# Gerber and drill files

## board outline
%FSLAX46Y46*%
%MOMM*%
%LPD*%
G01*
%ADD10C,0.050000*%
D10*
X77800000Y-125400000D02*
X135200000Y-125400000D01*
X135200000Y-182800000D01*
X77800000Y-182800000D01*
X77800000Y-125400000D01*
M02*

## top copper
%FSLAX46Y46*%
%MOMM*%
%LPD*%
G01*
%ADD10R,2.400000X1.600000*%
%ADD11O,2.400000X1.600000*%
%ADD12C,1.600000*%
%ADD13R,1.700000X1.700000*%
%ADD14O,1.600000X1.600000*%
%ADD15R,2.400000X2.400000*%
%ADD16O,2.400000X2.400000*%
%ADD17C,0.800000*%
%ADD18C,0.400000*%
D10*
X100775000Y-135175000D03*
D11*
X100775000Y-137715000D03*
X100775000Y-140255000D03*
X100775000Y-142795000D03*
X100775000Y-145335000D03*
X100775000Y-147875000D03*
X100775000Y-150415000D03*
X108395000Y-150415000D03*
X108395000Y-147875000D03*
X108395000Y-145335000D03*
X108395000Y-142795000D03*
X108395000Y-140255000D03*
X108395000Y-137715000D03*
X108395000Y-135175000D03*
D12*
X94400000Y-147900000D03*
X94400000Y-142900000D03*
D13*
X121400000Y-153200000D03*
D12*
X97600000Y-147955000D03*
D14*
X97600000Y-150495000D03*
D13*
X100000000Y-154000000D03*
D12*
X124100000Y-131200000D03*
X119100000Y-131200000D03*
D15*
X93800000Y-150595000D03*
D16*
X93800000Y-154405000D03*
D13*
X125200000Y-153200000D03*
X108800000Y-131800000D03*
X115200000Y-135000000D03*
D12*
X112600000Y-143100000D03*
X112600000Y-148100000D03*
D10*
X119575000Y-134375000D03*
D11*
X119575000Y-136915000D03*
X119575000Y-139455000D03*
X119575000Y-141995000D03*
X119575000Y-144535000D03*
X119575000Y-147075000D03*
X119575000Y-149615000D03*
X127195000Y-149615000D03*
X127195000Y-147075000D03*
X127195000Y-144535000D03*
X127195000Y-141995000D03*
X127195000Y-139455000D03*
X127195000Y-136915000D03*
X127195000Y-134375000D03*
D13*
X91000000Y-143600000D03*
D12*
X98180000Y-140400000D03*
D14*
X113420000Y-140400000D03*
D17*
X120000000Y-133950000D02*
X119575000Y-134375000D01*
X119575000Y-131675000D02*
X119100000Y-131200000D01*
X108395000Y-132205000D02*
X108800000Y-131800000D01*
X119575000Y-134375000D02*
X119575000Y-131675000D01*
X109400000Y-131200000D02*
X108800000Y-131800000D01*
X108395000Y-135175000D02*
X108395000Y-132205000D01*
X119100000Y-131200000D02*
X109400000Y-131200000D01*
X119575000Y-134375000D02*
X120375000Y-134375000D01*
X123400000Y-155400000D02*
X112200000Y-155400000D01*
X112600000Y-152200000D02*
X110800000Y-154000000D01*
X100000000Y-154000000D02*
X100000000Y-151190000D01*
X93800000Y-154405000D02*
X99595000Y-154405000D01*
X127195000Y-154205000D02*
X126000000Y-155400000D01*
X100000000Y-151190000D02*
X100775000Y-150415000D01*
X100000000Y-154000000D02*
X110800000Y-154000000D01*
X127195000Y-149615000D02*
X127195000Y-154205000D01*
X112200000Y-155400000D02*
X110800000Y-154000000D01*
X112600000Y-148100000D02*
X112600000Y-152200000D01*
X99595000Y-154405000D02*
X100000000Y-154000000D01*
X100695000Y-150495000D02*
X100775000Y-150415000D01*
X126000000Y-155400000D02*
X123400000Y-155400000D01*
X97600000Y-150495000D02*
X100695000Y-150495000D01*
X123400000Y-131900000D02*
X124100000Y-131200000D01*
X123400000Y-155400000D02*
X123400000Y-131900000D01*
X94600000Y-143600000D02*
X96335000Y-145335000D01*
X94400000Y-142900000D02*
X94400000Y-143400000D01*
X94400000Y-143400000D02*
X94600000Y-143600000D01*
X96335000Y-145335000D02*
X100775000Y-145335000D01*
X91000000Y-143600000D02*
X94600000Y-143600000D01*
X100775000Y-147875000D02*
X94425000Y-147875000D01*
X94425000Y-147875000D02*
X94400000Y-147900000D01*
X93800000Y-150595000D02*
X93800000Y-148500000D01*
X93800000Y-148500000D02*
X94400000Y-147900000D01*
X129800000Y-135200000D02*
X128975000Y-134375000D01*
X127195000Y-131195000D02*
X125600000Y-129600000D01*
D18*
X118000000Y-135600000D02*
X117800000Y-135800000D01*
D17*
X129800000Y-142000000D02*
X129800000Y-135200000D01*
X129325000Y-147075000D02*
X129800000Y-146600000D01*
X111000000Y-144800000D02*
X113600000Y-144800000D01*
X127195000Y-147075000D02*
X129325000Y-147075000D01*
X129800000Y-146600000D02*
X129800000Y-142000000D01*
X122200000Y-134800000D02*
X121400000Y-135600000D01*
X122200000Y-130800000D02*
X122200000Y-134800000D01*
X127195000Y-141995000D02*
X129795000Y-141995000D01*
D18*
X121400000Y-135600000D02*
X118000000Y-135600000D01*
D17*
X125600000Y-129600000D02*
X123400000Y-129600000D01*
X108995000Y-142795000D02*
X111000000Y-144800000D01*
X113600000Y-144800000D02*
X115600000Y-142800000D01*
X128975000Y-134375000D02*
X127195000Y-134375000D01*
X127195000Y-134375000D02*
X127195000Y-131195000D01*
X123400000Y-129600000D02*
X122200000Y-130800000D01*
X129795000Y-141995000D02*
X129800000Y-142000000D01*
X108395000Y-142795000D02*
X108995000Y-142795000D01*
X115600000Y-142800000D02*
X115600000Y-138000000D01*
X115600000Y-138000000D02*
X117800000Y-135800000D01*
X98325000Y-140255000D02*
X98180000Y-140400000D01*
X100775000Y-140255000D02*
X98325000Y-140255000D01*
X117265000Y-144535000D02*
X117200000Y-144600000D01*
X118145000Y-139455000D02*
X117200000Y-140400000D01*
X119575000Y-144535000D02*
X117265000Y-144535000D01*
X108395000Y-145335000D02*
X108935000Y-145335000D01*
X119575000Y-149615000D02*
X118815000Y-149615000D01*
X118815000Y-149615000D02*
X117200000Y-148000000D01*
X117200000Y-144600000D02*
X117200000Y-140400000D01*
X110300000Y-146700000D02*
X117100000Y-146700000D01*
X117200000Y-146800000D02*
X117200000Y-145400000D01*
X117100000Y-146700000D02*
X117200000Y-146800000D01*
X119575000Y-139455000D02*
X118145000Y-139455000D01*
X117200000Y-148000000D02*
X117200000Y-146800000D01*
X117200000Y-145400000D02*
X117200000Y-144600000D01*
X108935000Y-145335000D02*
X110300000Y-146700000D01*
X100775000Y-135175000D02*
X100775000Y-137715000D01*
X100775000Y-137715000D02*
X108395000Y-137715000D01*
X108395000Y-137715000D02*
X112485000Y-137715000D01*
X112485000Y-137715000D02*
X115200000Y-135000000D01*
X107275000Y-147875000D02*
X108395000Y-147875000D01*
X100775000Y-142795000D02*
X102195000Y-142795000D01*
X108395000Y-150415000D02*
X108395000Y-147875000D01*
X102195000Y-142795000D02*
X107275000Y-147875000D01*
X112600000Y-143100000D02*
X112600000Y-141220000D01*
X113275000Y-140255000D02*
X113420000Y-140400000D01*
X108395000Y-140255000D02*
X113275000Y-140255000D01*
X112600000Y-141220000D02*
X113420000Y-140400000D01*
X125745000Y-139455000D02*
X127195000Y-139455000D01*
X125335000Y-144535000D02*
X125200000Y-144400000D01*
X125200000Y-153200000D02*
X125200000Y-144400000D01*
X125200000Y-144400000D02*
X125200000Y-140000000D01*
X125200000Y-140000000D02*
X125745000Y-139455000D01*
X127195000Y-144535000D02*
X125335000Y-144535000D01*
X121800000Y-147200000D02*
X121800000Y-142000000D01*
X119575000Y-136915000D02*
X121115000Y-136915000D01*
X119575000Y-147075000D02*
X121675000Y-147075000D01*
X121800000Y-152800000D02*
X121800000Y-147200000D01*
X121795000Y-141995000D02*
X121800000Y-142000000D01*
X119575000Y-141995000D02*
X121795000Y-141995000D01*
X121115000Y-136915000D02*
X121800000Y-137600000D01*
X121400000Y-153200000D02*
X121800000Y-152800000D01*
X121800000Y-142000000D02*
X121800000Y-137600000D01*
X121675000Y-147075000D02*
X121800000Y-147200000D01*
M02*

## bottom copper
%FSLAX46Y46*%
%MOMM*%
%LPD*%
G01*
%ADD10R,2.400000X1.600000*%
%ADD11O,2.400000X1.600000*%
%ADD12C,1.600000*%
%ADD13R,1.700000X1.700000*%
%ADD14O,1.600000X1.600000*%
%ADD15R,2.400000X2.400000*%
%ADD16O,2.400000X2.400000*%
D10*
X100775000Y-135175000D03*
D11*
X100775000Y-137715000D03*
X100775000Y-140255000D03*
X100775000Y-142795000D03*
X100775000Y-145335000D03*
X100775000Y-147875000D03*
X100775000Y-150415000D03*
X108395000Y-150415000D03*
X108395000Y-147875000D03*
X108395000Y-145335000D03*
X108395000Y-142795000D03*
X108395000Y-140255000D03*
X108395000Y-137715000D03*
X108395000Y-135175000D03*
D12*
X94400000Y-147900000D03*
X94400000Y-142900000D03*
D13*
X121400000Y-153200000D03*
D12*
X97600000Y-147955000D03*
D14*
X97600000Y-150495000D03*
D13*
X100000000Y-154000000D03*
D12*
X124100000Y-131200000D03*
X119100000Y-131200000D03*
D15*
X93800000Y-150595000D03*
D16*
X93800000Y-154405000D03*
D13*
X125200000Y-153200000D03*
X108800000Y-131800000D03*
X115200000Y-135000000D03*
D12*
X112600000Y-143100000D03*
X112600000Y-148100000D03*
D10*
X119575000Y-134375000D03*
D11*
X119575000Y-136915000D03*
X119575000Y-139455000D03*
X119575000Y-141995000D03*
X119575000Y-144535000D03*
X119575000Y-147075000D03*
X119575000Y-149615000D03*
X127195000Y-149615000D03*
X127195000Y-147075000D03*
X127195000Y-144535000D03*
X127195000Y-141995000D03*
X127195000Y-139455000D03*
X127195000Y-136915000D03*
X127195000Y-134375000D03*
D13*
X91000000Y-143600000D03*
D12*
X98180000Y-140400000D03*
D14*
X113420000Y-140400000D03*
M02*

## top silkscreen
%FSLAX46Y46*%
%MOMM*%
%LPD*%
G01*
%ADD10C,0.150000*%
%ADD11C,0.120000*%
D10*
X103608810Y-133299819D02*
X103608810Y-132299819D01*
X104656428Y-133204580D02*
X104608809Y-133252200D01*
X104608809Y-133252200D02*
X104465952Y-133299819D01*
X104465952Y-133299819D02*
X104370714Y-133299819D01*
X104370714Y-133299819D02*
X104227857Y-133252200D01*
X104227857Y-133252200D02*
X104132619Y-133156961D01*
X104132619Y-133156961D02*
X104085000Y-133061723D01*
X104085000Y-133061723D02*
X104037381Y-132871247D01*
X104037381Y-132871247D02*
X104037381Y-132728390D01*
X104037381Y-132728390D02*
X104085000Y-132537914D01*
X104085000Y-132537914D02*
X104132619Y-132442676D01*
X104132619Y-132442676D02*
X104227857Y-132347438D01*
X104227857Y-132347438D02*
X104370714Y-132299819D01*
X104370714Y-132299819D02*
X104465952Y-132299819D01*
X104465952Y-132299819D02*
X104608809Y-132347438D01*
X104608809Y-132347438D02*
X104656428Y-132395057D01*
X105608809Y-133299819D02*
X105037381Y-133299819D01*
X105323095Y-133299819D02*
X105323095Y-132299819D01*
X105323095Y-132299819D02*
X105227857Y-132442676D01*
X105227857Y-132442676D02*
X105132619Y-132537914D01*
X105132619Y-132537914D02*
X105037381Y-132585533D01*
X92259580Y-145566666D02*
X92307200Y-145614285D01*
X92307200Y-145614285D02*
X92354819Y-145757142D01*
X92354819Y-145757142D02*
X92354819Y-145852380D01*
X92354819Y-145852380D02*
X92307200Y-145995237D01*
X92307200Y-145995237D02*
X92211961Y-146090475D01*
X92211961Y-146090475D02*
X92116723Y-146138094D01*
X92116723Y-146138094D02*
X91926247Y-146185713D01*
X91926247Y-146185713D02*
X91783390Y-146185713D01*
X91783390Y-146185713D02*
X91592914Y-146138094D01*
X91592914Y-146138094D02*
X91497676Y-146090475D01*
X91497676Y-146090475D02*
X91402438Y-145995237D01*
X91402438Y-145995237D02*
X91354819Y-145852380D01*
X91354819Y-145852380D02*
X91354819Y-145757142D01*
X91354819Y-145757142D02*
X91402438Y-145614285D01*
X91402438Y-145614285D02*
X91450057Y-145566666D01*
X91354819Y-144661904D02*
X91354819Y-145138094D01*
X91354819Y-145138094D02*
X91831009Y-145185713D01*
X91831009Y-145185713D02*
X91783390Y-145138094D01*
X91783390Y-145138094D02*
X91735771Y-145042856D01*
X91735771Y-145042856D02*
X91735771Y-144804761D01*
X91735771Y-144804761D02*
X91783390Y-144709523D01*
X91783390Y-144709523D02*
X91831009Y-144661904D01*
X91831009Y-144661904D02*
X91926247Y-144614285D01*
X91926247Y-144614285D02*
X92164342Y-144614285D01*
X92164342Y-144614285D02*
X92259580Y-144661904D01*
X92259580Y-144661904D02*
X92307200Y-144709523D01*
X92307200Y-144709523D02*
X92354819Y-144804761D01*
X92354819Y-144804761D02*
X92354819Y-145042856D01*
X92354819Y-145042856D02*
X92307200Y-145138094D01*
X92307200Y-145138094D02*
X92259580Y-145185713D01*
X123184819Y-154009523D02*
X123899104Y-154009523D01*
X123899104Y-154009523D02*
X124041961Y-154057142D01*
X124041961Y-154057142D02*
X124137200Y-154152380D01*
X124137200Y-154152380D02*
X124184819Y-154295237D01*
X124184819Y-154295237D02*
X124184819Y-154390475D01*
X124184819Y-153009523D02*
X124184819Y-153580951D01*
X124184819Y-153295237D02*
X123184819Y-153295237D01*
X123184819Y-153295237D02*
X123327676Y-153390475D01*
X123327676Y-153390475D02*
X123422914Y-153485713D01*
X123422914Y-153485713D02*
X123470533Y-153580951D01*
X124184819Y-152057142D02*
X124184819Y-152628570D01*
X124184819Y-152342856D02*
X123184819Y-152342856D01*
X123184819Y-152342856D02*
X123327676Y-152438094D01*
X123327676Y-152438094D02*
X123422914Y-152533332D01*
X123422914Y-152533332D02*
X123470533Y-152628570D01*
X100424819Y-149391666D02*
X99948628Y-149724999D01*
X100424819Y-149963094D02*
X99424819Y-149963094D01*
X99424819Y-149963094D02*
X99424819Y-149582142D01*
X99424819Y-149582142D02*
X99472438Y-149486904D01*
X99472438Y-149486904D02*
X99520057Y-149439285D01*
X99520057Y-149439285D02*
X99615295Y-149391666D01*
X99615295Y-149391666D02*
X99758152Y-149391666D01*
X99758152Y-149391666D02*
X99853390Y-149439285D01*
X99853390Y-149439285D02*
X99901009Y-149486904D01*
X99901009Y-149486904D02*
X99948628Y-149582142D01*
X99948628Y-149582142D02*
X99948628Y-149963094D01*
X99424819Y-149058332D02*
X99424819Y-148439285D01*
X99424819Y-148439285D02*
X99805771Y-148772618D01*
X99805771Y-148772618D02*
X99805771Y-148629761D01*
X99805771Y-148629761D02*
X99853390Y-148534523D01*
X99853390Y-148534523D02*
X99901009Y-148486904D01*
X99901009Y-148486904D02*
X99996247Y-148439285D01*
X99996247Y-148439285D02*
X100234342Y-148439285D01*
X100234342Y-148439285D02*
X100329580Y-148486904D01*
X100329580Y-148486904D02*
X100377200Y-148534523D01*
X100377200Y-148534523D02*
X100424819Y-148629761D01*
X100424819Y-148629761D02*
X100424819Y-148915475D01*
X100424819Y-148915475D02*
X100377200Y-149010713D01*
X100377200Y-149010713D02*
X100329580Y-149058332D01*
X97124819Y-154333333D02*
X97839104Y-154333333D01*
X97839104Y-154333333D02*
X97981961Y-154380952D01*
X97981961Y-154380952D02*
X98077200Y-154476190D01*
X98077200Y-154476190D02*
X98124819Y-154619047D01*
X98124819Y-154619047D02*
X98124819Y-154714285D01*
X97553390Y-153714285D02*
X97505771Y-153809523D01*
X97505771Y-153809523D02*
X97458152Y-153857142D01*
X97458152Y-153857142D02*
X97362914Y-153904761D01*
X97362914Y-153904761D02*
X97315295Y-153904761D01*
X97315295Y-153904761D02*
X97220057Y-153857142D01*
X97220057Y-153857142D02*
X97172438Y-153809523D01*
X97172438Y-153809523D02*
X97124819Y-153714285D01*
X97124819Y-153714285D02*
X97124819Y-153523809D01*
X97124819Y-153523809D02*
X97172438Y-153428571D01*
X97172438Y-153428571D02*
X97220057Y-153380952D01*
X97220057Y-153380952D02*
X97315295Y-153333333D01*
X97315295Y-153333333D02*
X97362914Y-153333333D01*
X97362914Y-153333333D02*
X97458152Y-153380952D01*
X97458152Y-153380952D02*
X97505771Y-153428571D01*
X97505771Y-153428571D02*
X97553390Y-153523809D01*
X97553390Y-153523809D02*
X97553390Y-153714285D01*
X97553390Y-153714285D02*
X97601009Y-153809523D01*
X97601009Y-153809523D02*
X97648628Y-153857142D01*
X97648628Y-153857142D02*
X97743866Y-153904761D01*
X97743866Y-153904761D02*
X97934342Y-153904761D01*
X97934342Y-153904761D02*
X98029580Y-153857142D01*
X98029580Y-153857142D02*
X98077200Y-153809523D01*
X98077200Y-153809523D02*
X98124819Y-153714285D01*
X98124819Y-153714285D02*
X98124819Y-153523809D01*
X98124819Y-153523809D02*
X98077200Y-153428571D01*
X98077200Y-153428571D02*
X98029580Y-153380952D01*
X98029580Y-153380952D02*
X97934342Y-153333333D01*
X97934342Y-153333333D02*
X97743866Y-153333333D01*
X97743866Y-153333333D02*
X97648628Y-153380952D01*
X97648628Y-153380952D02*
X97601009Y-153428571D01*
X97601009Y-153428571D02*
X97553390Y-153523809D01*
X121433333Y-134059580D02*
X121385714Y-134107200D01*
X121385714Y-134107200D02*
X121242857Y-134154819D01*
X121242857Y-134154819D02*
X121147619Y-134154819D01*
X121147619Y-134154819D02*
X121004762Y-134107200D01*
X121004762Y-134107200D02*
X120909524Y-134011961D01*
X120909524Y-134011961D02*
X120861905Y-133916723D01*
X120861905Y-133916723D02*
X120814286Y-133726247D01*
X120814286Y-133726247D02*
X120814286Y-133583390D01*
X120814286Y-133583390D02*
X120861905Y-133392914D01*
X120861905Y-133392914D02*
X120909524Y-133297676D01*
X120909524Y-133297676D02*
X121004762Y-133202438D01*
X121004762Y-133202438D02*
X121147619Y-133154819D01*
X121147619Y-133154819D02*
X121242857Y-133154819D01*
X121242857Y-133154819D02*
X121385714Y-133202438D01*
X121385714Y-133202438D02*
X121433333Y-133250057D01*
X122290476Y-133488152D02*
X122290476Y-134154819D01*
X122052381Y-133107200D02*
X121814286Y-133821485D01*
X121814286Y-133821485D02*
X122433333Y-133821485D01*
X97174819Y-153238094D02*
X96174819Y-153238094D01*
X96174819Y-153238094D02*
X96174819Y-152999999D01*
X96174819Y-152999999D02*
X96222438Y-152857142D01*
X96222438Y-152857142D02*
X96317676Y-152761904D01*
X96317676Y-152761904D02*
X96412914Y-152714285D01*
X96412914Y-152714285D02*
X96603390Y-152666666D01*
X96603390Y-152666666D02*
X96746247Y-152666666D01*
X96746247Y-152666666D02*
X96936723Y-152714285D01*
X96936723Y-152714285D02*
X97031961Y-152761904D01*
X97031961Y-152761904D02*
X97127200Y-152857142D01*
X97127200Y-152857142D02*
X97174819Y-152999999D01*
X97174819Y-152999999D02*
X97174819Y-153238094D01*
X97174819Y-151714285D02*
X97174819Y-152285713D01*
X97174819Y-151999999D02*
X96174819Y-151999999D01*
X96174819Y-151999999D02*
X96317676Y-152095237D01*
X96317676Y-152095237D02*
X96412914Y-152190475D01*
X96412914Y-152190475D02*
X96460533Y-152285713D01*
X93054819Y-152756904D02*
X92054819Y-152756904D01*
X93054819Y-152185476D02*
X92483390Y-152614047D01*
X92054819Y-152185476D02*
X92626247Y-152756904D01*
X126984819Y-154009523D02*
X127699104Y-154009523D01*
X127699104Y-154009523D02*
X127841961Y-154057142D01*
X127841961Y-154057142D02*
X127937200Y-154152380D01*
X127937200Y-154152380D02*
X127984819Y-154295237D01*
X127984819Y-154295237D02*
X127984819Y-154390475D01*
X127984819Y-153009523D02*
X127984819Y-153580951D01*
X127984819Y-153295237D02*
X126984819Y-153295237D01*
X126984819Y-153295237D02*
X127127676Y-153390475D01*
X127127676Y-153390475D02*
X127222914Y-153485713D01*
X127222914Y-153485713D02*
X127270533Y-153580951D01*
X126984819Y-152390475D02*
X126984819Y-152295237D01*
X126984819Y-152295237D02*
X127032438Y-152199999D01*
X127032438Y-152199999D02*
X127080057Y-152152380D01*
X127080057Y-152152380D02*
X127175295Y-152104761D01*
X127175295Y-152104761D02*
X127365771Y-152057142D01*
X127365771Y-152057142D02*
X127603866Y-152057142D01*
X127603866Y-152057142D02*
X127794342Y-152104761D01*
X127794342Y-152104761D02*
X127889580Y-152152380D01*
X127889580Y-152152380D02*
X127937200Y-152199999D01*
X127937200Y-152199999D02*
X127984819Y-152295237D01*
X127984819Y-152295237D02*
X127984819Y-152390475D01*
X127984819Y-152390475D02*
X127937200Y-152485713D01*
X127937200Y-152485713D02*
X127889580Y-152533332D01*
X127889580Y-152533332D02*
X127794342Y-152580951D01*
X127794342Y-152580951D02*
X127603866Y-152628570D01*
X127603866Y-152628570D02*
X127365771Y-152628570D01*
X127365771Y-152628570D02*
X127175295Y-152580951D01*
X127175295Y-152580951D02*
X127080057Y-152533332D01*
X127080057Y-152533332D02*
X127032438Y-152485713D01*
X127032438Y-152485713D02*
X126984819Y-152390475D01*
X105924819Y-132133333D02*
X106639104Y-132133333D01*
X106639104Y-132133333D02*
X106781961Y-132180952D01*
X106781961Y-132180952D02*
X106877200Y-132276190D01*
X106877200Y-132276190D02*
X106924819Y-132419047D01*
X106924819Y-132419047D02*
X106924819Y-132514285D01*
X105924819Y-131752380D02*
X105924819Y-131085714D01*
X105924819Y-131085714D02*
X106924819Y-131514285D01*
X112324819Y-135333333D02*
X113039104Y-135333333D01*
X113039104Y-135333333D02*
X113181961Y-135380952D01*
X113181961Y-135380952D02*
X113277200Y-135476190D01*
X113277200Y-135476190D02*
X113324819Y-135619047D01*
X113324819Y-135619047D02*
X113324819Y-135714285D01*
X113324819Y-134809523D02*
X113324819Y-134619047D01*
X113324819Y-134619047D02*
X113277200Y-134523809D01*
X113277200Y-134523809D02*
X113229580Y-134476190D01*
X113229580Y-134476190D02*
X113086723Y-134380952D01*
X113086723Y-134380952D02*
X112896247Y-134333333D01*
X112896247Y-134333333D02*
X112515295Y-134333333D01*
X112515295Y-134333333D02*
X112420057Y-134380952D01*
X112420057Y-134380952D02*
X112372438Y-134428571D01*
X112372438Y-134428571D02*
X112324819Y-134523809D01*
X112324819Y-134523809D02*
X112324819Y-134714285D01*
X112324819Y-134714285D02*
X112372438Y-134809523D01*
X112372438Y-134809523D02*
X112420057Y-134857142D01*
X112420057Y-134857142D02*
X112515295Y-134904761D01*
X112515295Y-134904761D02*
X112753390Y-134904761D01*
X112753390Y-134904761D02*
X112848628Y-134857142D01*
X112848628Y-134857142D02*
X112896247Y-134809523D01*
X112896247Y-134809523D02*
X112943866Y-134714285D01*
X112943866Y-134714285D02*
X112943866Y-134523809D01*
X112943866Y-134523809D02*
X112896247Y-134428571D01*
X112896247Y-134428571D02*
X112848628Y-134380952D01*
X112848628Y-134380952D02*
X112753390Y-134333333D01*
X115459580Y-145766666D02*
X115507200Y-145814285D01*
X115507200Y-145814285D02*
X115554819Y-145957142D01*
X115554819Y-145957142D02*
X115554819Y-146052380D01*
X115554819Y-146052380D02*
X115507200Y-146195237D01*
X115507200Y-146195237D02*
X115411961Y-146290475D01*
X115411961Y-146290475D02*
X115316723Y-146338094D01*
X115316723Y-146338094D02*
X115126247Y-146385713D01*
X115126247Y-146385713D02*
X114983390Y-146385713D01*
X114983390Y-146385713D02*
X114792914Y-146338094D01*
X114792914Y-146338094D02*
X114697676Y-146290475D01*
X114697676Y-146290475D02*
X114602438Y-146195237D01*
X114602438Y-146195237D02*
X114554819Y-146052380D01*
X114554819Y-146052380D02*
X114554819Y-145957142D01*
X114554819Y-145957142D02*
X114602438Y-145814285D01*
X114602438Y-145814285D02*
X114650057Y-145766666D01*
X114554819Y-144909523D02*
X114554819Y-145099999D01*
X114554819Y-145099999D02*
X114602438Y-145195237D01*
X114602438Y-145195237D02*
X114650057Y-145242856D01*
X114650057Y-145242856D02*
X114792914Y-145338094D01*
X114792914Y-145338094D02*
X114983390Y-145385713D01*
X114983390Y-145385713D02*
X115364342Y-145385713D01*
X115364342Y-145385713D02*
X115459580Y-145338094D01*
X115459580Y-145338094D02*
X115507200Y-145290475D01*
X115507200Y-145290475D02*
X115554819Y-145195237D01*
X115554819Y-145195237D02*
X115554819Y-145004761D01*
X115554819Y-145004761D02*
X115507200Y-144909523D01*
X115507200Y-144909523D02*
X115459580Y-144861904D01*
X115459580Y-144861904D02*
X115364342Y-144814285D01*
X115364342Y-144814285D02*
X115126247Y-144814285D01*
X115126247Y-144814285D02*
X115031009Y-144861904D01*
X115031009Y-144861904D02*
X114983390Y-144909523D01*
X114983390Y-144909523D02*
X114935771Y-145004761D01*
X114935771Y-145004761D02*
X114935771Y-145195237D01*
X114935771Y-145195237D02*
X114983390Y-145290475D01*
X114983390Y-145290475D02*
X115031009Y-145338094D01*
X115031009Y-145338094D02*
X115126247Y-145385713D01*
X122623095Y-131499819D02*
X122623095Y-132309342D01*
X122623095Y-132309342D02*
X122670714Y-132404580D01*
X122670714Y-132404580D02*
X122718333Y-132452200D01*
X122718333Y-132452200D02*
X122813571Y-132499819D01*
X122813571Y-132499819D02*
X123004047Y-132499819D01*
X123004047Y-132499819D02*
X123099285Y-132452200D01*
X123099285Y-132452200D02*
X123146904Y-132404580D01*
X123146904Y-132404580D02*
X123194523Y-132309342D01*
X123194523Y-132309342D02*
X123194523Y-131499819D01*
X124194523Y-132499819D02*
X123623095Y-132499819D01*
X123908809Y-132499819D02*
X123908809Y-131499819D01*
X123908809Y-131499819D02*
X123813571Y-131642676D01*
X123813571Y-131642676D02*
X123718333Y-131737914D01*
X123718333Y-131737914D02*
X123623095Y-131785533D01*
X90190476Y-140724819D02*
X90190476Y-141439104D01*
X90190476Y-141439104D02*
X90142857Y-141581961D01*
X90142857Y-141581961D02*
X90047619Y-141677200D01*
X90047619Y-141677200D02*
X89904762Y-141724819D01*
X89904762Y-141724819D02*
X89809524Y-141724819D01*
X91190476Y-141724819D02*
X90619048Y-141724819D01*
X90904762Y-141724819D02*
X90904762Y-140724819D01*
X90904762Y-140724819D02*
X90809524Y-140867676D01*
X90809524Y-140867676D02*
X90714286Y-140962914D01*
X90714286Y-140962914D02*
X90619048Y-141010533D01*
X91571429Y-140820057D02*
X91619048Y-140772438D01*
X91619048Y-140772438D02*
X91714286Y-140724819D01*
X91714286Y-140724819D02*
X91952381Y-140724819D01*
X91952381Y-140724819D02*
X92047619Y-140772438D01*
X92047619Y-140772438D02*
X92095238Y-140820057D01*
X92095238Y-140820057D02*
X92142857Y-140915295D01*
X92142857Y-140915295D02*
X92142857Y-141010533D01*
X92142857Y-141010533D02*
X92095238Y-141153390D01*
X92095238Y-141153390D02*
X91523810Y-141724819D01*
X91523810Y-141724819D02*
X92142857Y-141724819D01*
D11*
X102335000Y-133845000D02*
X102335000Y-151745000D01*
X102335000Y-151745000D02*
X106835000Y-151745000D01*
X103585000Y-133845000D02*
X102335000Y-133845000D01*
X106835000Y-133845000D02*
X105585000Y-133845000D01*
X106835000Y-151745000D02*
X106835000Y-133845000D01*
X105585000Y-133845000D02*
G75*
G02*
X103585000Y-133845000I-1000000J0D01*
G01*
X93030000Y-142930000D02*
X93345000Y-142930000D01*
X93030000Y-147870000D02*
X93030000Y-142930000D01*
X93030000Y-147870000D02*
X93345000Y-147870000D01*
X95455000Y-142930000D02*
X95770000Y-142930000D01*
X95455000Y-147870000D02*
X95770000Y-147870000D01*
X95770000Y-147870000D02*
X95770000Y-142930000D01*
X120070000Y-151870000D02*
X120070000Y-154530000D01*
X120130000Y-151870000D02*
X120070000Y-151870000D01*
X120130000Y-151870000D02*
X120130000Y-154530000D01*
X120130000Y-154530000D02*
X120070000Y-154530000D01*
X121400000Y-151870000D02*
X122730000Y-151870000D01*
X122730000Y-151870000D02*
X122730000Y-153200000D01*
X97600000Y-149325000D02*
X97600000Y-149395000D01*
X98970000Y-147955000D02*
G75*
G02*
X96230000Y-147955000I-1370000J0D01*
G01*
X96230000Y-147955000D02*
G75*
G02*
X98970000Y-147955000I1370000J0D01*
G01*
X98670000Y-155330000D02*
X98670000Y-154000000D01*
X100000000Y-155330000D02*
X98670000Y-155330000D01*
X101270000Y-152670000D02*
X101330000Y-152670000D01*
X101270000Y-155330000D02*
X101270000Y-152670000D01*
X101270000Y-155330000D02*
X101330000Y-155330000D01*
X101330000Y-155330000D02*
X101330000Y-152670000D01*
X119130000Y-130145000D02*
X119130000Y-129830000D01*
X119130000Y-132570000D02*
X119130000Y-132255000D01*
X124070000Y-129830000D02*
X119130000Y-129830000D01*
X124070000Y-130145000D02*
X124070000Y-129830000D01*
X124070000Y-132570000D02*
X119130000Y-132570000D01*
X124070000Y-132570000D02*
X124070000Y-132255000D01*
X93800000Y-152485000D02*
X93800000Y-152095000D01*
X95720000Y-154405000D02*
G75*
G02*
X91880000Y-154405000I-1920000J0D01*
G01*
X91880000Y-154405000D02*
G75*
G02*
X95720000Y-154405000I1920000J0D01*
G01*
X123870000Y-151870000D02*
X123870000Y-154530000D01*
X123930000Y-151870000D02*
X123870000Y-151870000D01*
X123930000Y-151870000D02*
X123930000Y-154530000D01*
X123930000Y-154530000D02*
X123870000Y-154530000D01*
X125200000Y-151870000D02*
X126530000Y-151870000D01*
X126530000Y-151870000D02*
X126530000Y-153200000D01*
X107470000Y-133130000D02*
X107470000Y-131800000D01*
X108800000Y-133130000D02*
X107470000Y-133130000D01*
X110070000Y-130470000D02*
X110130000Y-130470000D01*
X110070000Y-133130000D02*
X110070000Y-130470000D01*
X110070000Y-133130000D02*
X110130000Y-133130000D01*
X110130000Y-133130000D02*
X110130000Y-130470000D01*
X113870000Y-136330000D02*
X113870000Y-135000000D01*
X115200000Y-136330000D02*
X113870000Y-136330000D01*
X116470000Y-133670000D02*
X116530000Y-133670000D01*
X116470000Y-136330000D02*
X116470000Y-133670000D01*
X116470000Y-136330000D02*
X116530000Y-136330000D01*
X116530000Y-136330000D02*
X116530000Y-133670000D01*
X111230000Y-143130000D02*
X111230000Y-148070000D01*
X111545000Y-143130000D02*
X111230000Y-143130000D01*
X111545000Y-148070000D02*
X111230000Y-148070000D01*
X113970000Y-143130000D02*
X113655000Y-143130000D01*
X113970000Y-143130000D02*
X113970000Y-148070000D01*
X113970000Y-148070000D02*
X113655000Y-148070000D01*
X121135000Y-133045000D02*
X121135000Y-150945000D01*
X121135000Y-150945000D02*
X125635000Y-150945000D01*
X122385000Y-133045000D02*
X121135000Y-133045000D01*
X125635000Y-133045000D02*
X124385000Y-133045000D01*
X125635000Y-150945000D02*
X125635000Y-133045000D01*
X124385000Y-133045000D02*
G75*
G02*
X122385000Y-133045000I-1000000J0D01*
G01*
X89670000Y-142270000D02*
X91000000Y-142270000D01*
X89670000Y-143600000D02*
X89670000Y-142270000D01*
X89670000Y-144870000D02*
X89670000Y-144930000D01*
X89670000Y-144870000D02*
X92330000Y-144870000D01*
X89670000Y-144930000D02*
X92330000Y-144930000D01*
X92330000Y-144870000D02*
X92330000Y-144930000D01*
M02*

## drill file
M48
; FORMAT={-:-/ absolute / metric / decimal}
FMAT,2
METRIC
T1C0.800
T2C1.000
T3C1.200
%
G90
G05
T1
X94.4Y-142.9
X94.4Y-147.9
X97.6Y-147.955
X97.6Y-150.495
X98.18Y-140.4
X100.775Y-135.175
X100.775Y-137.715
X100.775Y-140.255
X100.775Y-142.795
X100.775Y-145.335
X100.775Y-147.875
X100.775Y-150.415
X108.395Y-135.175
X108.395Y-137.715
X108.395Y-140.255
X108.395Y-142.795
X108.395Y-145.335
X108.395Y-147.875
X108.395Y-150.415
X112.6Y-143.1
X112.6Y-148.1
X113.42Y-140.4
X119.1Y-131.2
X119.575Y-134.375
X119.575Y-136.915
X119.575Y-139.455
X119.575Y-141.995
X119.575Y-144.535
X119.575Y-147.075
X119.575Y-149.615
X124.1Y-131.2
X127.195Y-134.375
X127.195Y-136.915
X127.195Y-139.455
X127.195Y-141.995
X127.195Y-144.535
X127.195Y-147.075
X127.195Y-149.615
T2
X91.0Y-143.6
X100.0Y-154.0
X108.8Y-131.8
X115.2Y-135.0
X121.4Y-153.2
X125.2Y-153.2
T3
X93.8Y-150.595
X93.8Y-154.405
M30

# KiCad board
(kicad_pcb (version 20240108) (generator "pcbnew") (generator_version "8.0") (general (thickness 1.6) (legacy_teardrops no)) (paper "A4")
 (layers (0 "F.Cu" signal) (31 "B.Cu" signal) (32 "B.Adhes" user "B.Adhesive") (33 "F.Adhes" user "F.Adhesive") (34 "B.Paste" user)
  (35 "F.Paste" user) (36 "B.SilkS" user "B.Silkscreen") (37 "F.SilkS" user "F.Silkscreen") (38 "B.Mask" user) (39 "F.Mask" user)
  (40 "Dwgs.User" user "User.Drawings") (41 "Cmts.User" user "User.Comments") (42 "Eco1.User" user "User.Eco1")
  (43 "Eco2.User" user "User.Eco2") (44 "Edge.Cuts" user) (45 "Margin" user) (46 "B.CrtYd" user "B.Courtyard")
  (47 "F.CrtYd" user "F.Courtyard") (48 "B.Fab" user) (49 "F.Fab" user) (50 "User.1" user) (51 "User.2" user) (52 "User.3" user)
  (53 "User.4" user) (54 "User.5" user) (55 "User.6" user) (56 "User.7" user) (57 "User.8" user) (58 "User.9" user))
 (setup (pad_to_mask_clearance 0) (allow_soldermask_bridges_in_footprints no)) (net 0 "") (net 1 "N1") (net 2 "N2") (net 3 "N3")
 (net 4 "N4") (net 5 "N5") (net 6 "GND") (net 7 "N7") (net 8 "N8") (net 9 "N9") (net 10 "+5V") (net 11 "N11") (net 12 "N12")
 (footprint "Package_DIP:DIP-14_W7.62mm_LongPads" (layer "F.Cu") (at 100.775 135.175)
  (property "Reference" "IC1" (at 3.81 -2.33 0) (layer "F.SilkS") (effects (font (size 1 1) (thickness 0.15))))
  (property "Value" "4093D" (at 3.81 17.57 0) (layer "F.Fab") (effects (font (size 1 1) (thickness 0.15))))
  (fp_line (start 1.56 -1.33) (end 1.56 16.57) (stroke (width 0.12) (type solid)) (layer "F.SilkS"))
  (fp_line (start 1.56 16.57) (end 6.06 16.57) (stroke (width 0.12) (type solid)) (layer "F.SilkS"))
  (fp_line (start 2.81 -1.33) (end 1.56 -1.33) (stroke (width 0.12) (type solid)) (layer "F.SilkS"))
  (fp_line (start 6.06 -1.33) (end 4.81 -1.33) (stroke (width 0.12) (type solid)) (layer "F.SilkS"))
  (fp_line (start 6.06 16.57) (end 6.06 -1.33) (stroke (width 0.12) (type solid)) (layer "F.SilkS"))
  (fp_arc (start 4.81 -1.33) (mid 3.81 -0.33) (end 2.81 -1.33) (stroke (width 0.12) (type solid)) (layer "F.SilkS"))
  (pad "1" thru_hole rect (at 0 0) (size 2.4 1.6) (drill 0.8) (layers "*.Cu" "*.Mask") (remove_unused_layers no) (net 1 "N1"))
  (pad "2" thru_hole oval (at 0 2.54) (size 2.4 1.6) (drill 0.8) (layers "*.Cu" "*.Mask") (remove_unused_layers no) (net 1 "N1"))
  (pad "3" thru_hole oval (at 0 5.08) (size 2.4 1.6) (drill 0.8) (layers "*.Cu" "*.Mask") (remove_unused_layers no) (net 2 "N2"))
  (pad "4" thru_hole oval (at 0 7.62) (size 2.4 1.6) (drill 0.8) (layers "*.Cu" "*.Mask") (remove_unused_layers no) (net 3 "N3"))
  (pad "5" thru_hole oval (at 0 10.16) (size 2.4 1.6) (drill 0.8) (layers "*.Cu" "*.Mask") (remove_unused_layers no) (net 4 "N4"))
  (pad "6" thru_hole oval (at 0 12.7) (size 2.4 1.6) (drill 0.8) (layers "*.Cu" "*.Mask") (remove_unused_layers no) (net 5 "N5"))
  (pad "7" thru_hole oval (at 0 15.24) (size 2.4 1.6) (drill 0.8) (layers "*.Cu" "*.Mask") (remove_unused_layers no) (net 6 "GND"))
  (pad "8" thru_hole oval (at 7.62 15.24) (size 2.4 1.6) (drill 0.8) (layers "*.Cu" "*.Mask") (remove_unused_layers no) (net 3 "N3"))
  (pad "9" thru_hole oval (at 7.62 12.7) (size 2.4 1.6) (drill 0.8) (layers "*.Cu" "*.Mask") (remove_unused_layers no) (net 3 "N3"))
  (pad "10" thru_hole oval (at 7.62 10.16) (size 2.4 1.6) (drill 0.8) (layers "*.Cu" "*.Mask") (remove_unused_layers no) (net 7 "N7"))
  (pad "11" thru_hole oval (at 7.62 7.62) (size 2.4 1.6) (drill 0.8) (layers "*.Cu" "*.Mask") (remove_unused_layers no) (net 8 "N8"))
  (pad "12" thru_hole oval (at 7.62 5.08) (size 2.4 1.6) (drill 0.8) (layers "*.Cu" "*.Mask") (remove_unused_layers no) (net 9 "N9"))
  (pad "13" thru_hole oval (at 7.62 2.54) (size 2.4 1.6) (drill 0.8) (layers "*.Cu" "*.Mask") (remove_unused_layers no) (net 1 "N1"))
  (pad "14" thru_hole oval (at 7.62 0) (size 2.4 1.6) (drill 0.8) (layers "*.Cu" "*.Mask") (remove_unused_layers no) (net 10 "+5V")))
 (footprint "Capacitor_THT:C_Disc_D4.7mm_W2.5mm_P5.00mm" (layer "F.Cu") (at 94.4 147.9 90)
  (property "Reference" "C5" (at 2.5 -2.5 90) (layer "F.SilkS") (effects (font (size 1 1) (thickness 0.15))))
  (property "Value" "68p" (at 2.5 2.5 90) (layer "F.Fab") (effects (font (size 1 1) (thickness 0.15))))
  (fp_line (start 4.97 -1.37) (end 4.97 -1.055) (stroke (width 0.12) (type solid)) (layer "F.SilkS"))
  (fp_line (start 0.03 -1.37) (end 4.97 -1.37) (stroke (width 0.12) (type solid)) (layer "F.SilkS"))
  (fp_line (start 0.03 -1.37) (end 0.03 -1.055) (stroke (width 0.12) (type solid)) (layer "F.SilkS"))
  (fp_line (start 4.97 1.055) (end 4.97 1.37) (stroke (width 0.12) (type solid)) (layer "F.SilkS"))
  (fp_line (start 0.03 1.055) (end 0.03 1.37) (stroke (width 0.12) (type solid)) (layer "F.SilkS"))
  (fp_line (start 0.03 1.37) (end 4.97 1.37) (stroke (width 0.12) (type solid)) (layer "F.SilkS"))
  (pad "1" thru_hole circle (at 0 0 90) (size 1.6 1.6) (drill 0.8) (layers "*.Cu" "*.Mask") (remove_unused_layers no) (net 5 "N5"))
  (pad "2" thru_hole circle (at 5 0 90) (size 1.6 1.6) (drill 0.8) (layers "*.Cu" "*.Mask") (remove_unused_layers no) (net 4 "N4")))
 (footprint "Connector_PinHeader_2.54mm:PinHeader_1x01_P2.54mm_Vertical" (layer "F.Cu") (at 121.4 153.2 -90)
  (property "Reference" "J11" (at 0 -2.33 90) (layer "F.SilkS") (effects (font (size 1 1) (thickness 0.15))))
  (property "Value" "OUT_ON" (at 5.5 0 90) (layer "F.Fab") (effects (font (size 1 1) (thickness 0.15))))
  (fp_line (start -1.33 1.33) (end 1.33 1.33) (stroke (width 0.12) (type solid)) (layer "F.SilkS"))
  (fp_line (start -1.33 1.27) (end -1.33 1.33) (stroke (width 0.12) (type solid)) (layer "F.SilkS"))
  (fp_line (start -1.33 1.27) (end 1.33 1.27) (stroke (width 0.12) (type solid)) (layer "F.SilkS"))
  (fp_line (start 1.33 1.27) (end 1.33 1.33) (stroke (width 0.12) (type solid)) (layer "F.SilkS"))
  (fp_line (start -1.33 0) (end -1.33 -1.33) (stroke (width 0.12) (type solid)) (layer "F.SilkS"))
  (fp_line (start -1.33 -1.33) (end 0 -1.33) (stroke (width 0.12) (type solid)) (layer "F.SilkS"))
  (pad "1" thru_hole rect (at 0 0 270) (size 1.7 1.7) (drill 1) (layers "*.Cu" "*.Mask") (remove_unused_layers no) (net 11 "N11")))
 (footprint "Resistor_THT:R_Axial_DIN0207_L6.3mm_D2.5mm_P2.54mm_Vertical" (layer "F.Cu") (at 97.6 147.955 -90)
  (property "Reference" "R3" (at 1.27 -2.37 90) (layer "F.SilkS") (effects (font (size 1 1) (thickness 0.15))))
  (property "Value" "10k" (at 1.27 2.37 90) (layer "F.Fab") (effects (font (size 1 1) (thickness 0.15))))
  (fp_line (start 1.37 0) (end 1.44 0) (stroke (width 0.12) (type solid)) (layer "F.SilkS"))
  (fp_circle (center 0 0) (end 1.37 0) (stroke (width 0.12) (type solid)) (fill none) (layer "F.SilkS"))
  (pad "1" thru_hole circle (at 0 0 270) (size 1.6 1.6) (drill 0.8) (layers "*.Cu" "*.Mask") (remove_unused_layers no) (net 5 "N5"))
  (pad "2" thru_hole oval (at 2.54 0 270) (size 1.6 1.6) (drill 0.8) (layers "*.Cu" "*.Mask") (remove_unused_layers no) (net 6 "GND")))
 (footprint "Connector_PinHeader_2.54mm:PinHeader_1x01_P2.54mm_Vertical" (layer "F.Cu") (at 100 154 90)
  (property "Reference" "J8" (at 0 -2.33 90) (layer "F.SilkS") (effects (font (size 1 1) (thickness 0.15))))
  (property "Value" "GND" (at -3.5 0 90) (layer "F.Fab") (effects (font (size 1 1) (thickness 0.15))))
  (fp_line (start -1.33 -1.33) (end 0 -1.33) (stroke (width 0.12) (type solid)) (layer "F.SilkS"))
  (fp_line (start -1.33 0) (end -1.33 -1.33) (stroke (width 0.12) (type solid)) (layer "F.SilkS"))
  (fp_line (start 1.33 1.27) (end 1.33 1.33) (stroke (width 0.12) (type solid)) (layer "F.SilkS"))
  (fp_line (start -1.33 1.27) (end 1.33 1.27) (stroke (width 0.12) (type solid)) (layer "F.SilkS"))
  (fp_line (start -1.33 1.27) (end -1.33 1.33) (stroke (width 0.12) (type solid)) (layer "F.SilkS"))
  (fp_line (start -1.33 1.33) (end 1.33 1.33) (stroke (width 0.12) (type solid)) (layer "F.SilkS"))
  (pad "1" thru_hole rect (at 0 0 90) (size 1.7 1.7) (drill 1) (layers "*.Cu" "*.Mask") (remove_unused_layers no) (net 6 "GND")))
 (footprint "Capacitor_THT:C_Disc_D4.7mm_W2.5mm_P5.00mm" (layer "F.Cu") (at 124.1 131.2 180)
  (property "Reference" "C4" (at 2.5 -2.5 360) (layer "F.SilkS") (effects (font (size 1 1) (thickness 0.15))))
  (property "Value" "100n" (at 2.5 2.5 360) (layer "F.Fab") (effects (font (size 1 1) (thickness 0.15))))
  (fp_line (start 4.97 1.055) (end 4.97 1.37) (stroke (width 0.12) (type solid)) (layer "F.SilkS"))
  (fp_line (start 4.97 -1.37) (end 4.97 -1.055) (stroke (width 0.12) (type solid)) (layer "F.SilkS"))
  (fp_line (start 0.03 1.37) (end 4.97 1.37) (stroke (width 0.12) (type solid)) (layer "F.SilkS"))
  (fp_line (start 0.03 1.055) (end 0.03 1.37) (stroke (width 0.12) (type solid)) (layer "F.SilkS"))
  (fp_line (start 0.03 -1.37) (end 4.97 -1.37) (stroke (width 0.12) (type solid)) (layer "F.SilkS"))
  (fp_line (start 0.03 -1.37) (end 0.03 -1.055) (stroke (width 0.12) (type solid)) (layer "F.SilkS"))
  (pad "1" thru_hole circle (at 0 0 180) (size 1.6 1.6) (drill 0.8) (layers "*.Cu" "*.Mask") (remove_unused_layers no) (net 6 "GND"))
  (pad "2" thru_hole circle (at 5 0 180) (size 1.6 1.6) (drill 0.8) (layers "*.Cu" "*.Mask") (remove_unused_layers no) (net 10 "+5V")))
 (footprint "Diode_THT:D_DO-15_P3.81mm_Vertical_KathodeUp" (layer "F.Cu") (at 93.8 150.595 -90)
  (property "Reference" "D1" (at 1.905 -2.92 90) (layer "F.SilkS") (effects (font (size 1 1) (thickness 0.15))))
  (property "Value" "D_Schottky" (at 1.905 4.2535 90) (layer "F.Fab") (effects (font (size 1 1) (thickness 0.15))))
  (fp_line (start 1.89 0) (end 1.5 0) (stroke (width 0.12) (type solid)) (layer "F.SilkS"))
  (fp_circle (center 3.81 0) (end 5.73 0) (stroke (width 0.12) (type solid)) (fill none) (layer "F.SilkS"))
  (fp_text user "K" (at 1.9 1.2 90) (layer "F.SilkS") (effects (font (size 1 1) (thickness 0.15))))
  (pad "1" thru_hole rect (at 0 0 270) (size 2.4 2.4) (drill 1.2) (layers "*.Cu" "*.Mask") (remove_unused_layers no) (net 5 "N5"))
  (pad "2" thru_hole oval (at 3.81 0 270) (size 2.4 2.4) (drill 1.2) (layers "*.Cu" "*.Mask") (remove_unused_layers no) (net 6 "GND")))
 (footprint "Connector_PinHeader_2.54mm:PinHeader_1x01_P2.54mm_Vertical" (layer "F.Cu") (at 125.2 153.2 -90)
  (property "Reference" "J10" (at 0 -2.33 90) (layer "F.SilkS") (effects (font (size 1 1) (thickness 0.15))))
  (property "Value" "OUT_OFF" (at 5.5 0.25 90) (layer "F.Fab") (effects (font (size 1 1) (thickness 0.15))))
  (fp_line (start -1.33 1.33) (end 1.33 1.33) (stroke (width 0.12) (type solid)) (layer "F.SilkS"))
  (fp_line (start -1.33 1.27) (end -1.33 1.33) (stroke (width 0.12) (type solid)) (layer "F.SilkS"))
  (fp_line (start -1.33 1.27) (end 1.33 1.27) (stroke (width 0.12) (type solid)) (layer "F.SilkS"))
  (fp_line (start 1.33 1.27) (end 1.33 1.33) (stroke (width 0.12) (type solid)) (layer "F.SilkS"))
  (fp_line (start -1.33 0) (end -1.33 -1.33) (stroke (width 0.12) (type solid)) (layer "F.SilkS"))
  (fp_line (start -1.33 -1.33) (end 0 -1.33) (stroke (width 0.12) (type solid)) (layer "F.SilkS"))
  (pad "1" thru_hole rect (at 0 0 270) (size 1.7 1.7) (drill 1) (layers "*.Cu" "*.Mask") (remove_unused_layers no) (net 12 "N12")))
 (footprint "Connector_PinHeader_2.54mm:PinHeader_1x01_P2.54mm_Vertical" (layer "F.Cu") (at 108.8 131.8 90)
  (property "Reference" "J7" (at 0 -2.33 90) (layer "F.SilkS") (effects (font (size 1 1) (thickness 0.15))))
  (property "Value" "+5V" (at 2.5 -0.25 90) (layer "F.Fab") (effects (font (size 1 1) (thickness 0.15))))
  (fp_line (start -1.33 -1.33) (end 0 -1.33) (stroke (width 0.12) (type solid)) (layer "F.SilkS"))
  (fp_line (start -1.33 0) (end -1.33 -1.33) (stroke (width 0.12) (type solid)) (layer "F.SilkS"))
  (fp_line (start 1.33 1.27) (end 1.33 1.33) (stroke (width 0.12) (type solid)) (layer "F.SilkS"))
  (fp_line (start -1.33 1.27) (end 1.33 1.27) (stroke (width 0.12) (type solid)) (layer "F.SilkS"))
  (fp_line (start -1.33 1.27) (end -1.33 1.33) (stroke (width 0.12) (type solid)) (layer "F.SilkS"))
  (fp_line (start -1.33 1.33) (end 1.33 1.33) (stroke (width 0.12) (type solid)) (layer "F.SilkS"))
  (pad "1" thru_hole rect (at 0 0 90) (size 1.7 1.7) (drill 1) (layers "*.Cu" "*.Mask") (remove_unused_layers no) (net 10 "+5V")))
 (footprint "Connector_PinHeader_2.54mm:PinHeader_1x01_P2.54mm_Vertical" (layer "F.Cu") (at 115.2 135 90)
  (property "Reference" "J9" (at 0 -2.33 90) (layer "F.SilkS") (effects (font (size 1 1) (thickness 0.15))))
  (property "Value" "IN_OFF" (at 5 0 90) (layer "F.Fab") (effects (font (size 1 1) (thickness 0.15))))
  (fp_line (start -1.33 -1.33) (end 0 -1.33) (stroke (width 0.12) (type solid)) (layer "F.SilkS"))
  (fp_line (start -1.33 0) (end -1.33 -1.33) (stroke (width 0.12) (type solid)) (layer "F.SilkS"))
  (fp_line (start 1.33 1.27) (end 1.33 1.33) (stroke (width 0.12) (type solid)) (layer "F.SilkS"))
  (fp_line (start -1.33 1.27) (end 1.33 1.27) (stroke (width 0.12) (type solid)) (layer "F.SilkS"))
  (fp_line (start -1.33 1.27) (end -1.33 1.33) (stroke (width 0.12) (type solid)) (layer "F.SilkS"))
  (fp_line (start -1.33 1.33) (end 1.33 1.33) (stroke (width 0.12) (type solid)) (layer "F.SilkS"))
  (pad "1" thru_hole rect (at 0 0 90) (size 1.7 1.7) (drill 1) (layers "*.Cu" "*.Mask") (remove_unused_layers no) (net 1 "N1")))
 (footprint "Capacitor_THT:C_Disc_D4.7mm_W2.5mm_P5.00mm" (layer "F.Cu") (at 112.6 143.1 -90)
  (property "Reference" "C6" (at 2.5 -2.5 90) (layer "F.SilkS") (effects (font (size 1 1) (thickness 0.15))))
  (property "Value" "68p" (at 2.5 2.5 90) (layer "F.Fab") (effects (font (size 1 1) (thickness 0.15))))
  (fp_line (start 0.03 1.37) (end 4.97 1.37) (stroke (width 0.12) (type solid)) (layer "F.SilkS"))
  (fp_line (start 0.03 1.055) (end 0.03 1.37) (stroke (width 0.12) (type solid)) (layer "F.SilkS"))
  (fp_line (start 4.97 1.055) (end 4.97 1.37) (stroke (width 0.12) (type solid)) (layer "F.SilkS"))
  (fp_line (start 0.03 -1.37) (end 0.03 -1.055) (stroke (width 0.12) (type solid)) (layer "F.SilkS"))
  (fp_line (start 0.03 -1.37) (end 4.97 -1.37) (stroke (width 0.12) (type solid)) (layer "F.SilkS"))
  (fp_line (start 4.97 -1.37) (end 4.97 -1.055) (stroke (width 0.12) (type solid)) (layer "F.SilkS"))
  (pad "1" thru_hole circle (at 0 0 270) (size 1.6 1.6) (drill 0.8) (layers "*.Cu" "*.Mask") (remove_unused_layers no) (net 9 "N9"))
  (pad "2" thru_hole circle (at 5 0 270) (size 1.6 1.6) (drill 0.8) (layers "*.Cu" "*.Mask") (remove_unused_layers no) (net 6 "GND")))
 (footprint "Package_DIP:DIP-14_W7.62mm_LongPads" (layer "F.Cu") (at 119.575 134.375)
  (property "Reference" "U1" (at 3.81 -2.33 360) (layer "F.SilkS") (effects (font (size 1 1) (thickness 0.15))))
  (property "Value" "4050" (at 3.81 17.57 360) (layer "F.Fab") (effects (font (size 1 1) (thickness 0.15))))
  (fp_line (start 1.56 -1.33) (end 1.56 16.57) (stroke (width 0.12) (type solid)) (layer "F.SilkS"))
  (fp_line (start 1.56 16.57) (end 6.06 16.57) (stroke (width 0.12) (type solid)) (layer "F.SilkS"))
  (fp_line (start 2.81 -1.33) (end 1.56 -1.33) (stroke (width 0.12) (type solid)) (layer "F.SilkS"))
  (fp_line (start 6.06 -1.33) (end 4.81 -1.33) (stroke (width 0.12) (type solid)) (layer "F.SilkS"))
  (fp_line (start 6.06 16.57) (end 6.06 -1.33) (stroke (width 0.12) (type solid)) (layer "F.SilkS"))
  (fp_arc (start 4.81 -1.33) (mid 3.81 -0.33) (end 2.81 -1.33) (stroke (width 0.12) (type solid)) (layer "F.SilkS"))
  (pad "1" thru_hole rect (at 0 0) (size 2.4 1.6) (drill 0.8) (layers "*.Cu" "*.Mask") (remove_unused_layers no) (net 10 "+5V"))
  (pad "2" thru_hole oval (at 0 2.54) (size 2.4 1.6) (drill 0.8) (layers "*.Cu" "*.Mask") (remove_unused_layers no) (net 11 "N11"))
  (pad "3" thru_hole oval (at 0 5.08) (size 2.4 1.6) (drill 0.8) (layers "*.Cu" "*.Mask") (remove_unused_layers no) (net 7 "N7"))
  (pad "4" thru_hole oval (at 0 7.62) (size 2.4 1.6) (drill 0.8) (layers "*.Cu" "*.Mask") (remove_unused_layers no) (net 11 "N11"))
  (pad "5" thru_hole oval (at 0 10.16) (size 2.4 1.6) (drill 0.8) (layers "*.Cu" "*.Mask") (remove_unused_layers no) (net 7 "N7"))
  (pad "6" thru_hole oval (at 0 12.7) (size 2.4 1.6) (drill 0.8) (layers "*.Cu" "*.Mask") (remove_unused_layers no) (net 11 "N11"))
  (pad "7" thru_hole oval (at 0 15.24) (size 2.4 1.6) (drill 0.8) (layers "*.Cu" "*.Mask") (remove_unused_layers no) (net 7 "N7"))
  (pad "8" thru_hole oval (at 7.62 15.24) (size 2.4 1.6) (drill 0.8) (layers "*.Cu" "*.Mask") (remove_unused_layers no) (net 6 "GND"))
  (pad "9" thru_hole oval (at 7.62 12.7) (size 2.4 1.6) (drill 0.8) (layers "*.Cu" "*.Mask") (remove_unused_layers no) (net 8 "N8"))
  (pad "10" thru_hole oval (at 7.62 10.16) (size 2.4 1.6) (drill 0.8) (layers "*.Cu" "*.Mask") (remove_unused_layers no) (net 12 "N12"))
  (pad "11" thru_hole oval (at 7.62 7.62) (size 2.4 1.6) (drill 0.8) (layers "*.Cu" "*.Mask") (remove_unused_layers no) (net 8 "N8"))
  (pad "12" thru_hole oval (at 7.62 5.08) (size 2.4 1.6) (drill 0.8) (layers "*.Cu" "*.Mask") (remove_unused_layers no) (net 12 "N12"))
  (pad "13" thru_hole oval (at 7.62 2.54) (size 2.4 1.6) (drill 0.8) (layers "*.Cu" "*.Mask") (remove_unused_layers no))
  (pad "14" thru_hole oval (at 7.62 0) (size 2.4 1.6) (drill 0.8) (layers "*.Cu" "*.Mask") (remove_unused_layers no) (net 8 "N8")))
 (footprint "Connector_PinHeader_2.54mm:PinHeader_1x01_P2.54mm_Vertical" (layer "F.Cu") (at 91 143.6)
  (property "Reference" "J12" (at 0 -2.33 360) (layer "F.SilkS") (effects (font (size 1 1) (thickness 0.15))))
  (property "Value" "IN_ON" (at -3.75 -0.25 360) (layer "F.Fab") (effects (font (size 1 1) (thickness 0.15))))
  (fp_line (start -1.33 -1.33) (end 0 -1.33) (stroke (width 0.12) (type solid)) (layer "F.SilkS"))
  (fp_line (start -1.33 0) (end -1.33 -1.33) (stroke (width 0.12) (type solid)) (layer "F.SilkS"))
  (fp_line (start -1.33 1.27) (end -1.33 1.33) (stroke (width 0.12) (type solid)) (layer "F.SilkS"))
  (fp_line (start -1.33 1.27) (end 1.33 1.27) (stroke (width 0.12) (type solid)) (layer "F.SilkS"))
  (fp_line (start -1.33 1.33) (end 1.33 1.33) (stroke (width 0.12) (type solid)) (layer "F.SilkS"))
  (fp_line (start 1.33 1.27) (end 1.33 1.33) (stroke (width 0.12) (type solid)) (layer "F.SilkS"))
  (pad "1" thru_hole rect (at 0 0) (size 1.7 1.7) (drill 1) (layers "*.Cu" "*.Mask") (remove_unused_layers no) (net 4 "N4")))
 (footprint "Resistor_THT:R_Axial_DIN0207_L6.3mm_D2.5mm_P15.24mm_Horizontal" (layer "B.Cu") (at 98.18 140.4)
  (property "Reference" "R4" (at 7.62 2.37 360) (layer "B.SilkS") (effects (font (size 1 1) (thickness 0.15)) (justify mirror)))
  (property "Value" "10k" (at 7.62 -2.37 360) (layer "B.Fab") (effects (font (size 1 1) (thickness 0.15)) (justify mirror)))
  (pad "1" thru_hole circle (at 0 0) (size 1.6 1.6) (drill 0.8) (layers "*.Cu" "*.Mask") (remove_unused_layers no) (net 2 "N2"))
  (pad "2" thru_hole oval (at 15.24 0) (size 1.6 1.6) (drill 0.8) (layers "*.Cu" "*.Mask") (remove_unused_layers no) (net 9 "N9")))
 (gr_rect (start 77.8 125.4) (end 135.2 182.8) (stroke (width 0.05) (type default)) (fill none) (layer "Edge.Cuts"))
 (segment (start 120 133.95) (end 119.575 134.375) (width 0.8) (layer "F.Cu") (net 10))
 (segment (start 119.575 131.675) (end 119.1 131.2) (width 0.8) (layer "F.Cu") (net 10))
 (segment (start 108.395 132.205) (end 108.8 131.8) (width 0.8) (layer "F.Cu") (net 10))
 (segment (start 119.575 134.375) (end 119.575 131.675) (width 0.8) (layer "F.Cu") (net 10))
 (segment (start 109.4 131.2) (end 108.8 131.8) (width 0.8) (layer "F.Cu") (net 10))
 (segment (start 108.395 135.175) (end 108.395 132.205) (width 0.8) (layer "F.Cu") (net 10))
 (segment (start 119.1 131.2) (end 109.4 131.2) (width 0.8) (layer "F.Cu") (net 10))
 (segment (start 119.575 134.375) (end 120.375 134.375) (width 0.8) (layer "F.Cu") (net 10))
 (segment (start 123.4 155.4) (end 112.2 155.4) (width 0.8) (layer "F.Cu") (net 6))
 (segment (start 112.6 152.2) (end 110.8 154) (width 0.8) (layer "F.Cu") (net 6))
 (segment (start 100 154) (end 100 151.19) (width 0.8) (layer "F.Cu") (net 6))
 (segment (start 93.8 154.405) (end 99.595 154.405) (width 0.8) (layer "F.Cu") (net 6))
 (segment (start 127.195 154.205) (end 126 155.4) (width 0.8) (layer "F.Cu") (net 6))
 (segment (start 100 151.19) (end 100.775 150.415) (width 0.8) (layer "F.Cu") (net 6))
 (segment (start 100 154) (end 110.8 154) (width 0.8) (layer "F.Cu") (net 6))
 (segment (start 127.195 149.615) (end 127.195 154.205) (width 0.8) (layer "F.Cu") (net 6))
 (segment (start 112.2 155.4) (end 110.8 154) (width 0.8) (layer "F.Cu") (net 6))
 (segment (start 112.6 148.1) (end 112.6 152.2) (width 0.8) (layer "F.Cu") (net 6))
 (segment (start 99.595 154.405) (end 100 154) (width 0.8) (layer "F.Cu") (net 6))
 (segment (start 100.695 150.495) (end 100.775 150.415) (width 0.8) (layer "F.Cu") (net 6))
 (segment (start 126 155.4) (end 123.4 155.4) (width 0.8) (layer "F.Cu") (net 6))
 (segment (start 97.6 150.495) (end 100.695 150.495) (width 0.8) (layer "F.Cu") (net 6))
 (segment (start 123.4 131.9) (end 124.1 131.2) (width 0.8) (layer "F.Cu") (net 6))
 (segment (start 123.4 155.4) (end 123.4 131.9) (width 0.8) (layer "F.Cu") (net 6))
 (segment (start 94.6 143.6) (end 96.335 145.335) (width 0.8) (layer "F.Cu") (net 4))
 (segment (start 94.4 142.9) (end 94.4 143.4) (width 0.8) (layer "F.Cu") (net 4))
 (segment (start 94.4 143.4) (end 94.6 143.6) (width 0.8) (layer "F.Cu") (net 4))
 (segment (start 96.335 145.335) (end 100.775 145.335) (width 0.8) (layer "F.Cu") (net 4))
 (segment (start 91 143.6) (end 94.6 143.6) (width 0.8) (layer "F.Cu") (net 4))
 (segment (start 100.775 147.875) (end 94.425 147.875) (width 0.8) (layer "F.Cu") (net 5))
 (segment (start 94.425 147.875) (end 94.4 147.9) (width 0.8) (layer "F.Cu") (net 5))
 (segment (start 93.8 150.595) (end 93.8 148.5) (width 0.8) (layer "F.Cu") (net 5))
 (segment (start 93.8 148.5) (end 94.4 147.9) (width 0.8) (layer "F.Cu") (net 5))
 (segment (start 129.8 135.2) (end 128.975 134.375) (width 0.8) (layer "F.Cu") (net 8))
 (segment (start 127.195 131.195) (end 125.6 129.6) (width 0.8) (layer "F.Cu") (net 8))
 (segment (start 118 135.6) (end 117.8 135.8) (width 0.4) (layer "F.Cu") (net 8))
 (segment (start 129.8 142) (end 129.8 135.2) (width 0.8) (layer "F.Cu") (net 8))
 (segment (start 129.325 147.075) (end 129.8 146.6) (width 0.8) (layer "F.Cu") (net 8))
 (segment (start 111 144.8) (end 113.6 144.8) (width 0.8) (layer "F.Cu") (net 8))
 (segment (start 127.195 147.075) (end 129.325 147.075) (width 0.8) (layer "F.Cu") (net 8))
 (segment (start 129.8 146.6) (end 129.8 142) (width 0.8) (layer "F.Cu") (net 8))
 (segment (start 122.2 134.8) (end 121.4 135.6) (width 0.8) (layer "F.Cu") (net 8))
 (segment (start 122.2 130.8) (end 122.2 134.8) (width 0.8) (layer "F.Cu") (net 8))
 (segment (start 127.195 141.995) (end 129.795 141.995) (width 0.8) (layer "F.Cu") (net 8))
 (segment (start 121.4 135.6) (end 118 135.6) (width 0.4) (layer "F.Cu") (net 8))
 (segment (start 125.6 129.6) (end 123.4 129.6) (width 0.8) (layer "F.Cu") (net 8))
 (segment (start 108.995 142.795) (end 111 144.8) (width 0.8) (layer "F.Cu") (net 8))
 (segment (start 113.6 144.8) (end 115.6 142.8) (width 0.8) (layer "F.Cu") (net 8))
 (segment (start 128.975 134.375) (end 127.195 134.375) (width 0.8) (layer "F.Cu") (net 8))
 (segment (start 127.195 134.375) (end 127.195 131.195) (width 0.8) (layer "F.Cu") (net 8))
 (segment (start 123.4 129.6) (end 122.2 130.8) (width 0.8) (layer "F.Cu") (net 8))
 (segment (start 129.795 141.995) (end 129.8 142) (width 0.8) (layer "F.Cu") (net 8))
 (segment (start 108.395 142.795) (end 108.995 142.795) (width 0.8) (layer "F.Cu") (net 8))
 (segment (start 115.6 142.8) (end 115.6 138) (width 0.8) (layer "F.Cu") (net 8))
 (segment (start 115.6 138) (end 117.8 135.8) (width 0.8) (layer "F.Cu") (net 8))
 (segment (start 98.325 140.255) (end 98.18 140.4) (width 0.8) (layer "F.Cu") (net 2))
 (segment (start 100.775 140.255) (end 98.325 140.255) (width 0.8) (layer "F.Cu") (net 2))
 (segment (start 117.265 144.535) (end 117.2 144.6) (width 0.8) (layer "F.Cu") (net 7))
 (segment (start 118.145 139.455) (end 117.2 140.4) (width 0.8) (layer "F.Cu") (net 7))
 (segment (start 119.575 144.535) (end 117.265 144.535) (width 0.8) (layer "F.Cu") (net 7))
 (segment (start 108.395 145.335) (end 108.935 145.335) (width 0.8) (layer "F.Cu") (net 7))
 (segment (start 119.575 149.615) (end 118.815 149.615) (width 0.8) (layer "F.Cu") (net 7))
 (segment (start 118.815 149.615) (end 117.2 148) (width 0.8) (layer "F.Cu") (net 7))
 (segment (start 117.2 144.6) (end 117.2 140.4) (width 0.8) (layer "F.Cu") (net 7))
 (segment (start 110.3 146.7) (end 117.1 146.7) (width 0.8) (layer "F.Cu") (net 7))
 (segment (start 117.2 146.8) (end 117.2 145.4) (width 0.8) (layer "F.Cu") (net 7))
 (segment (start 117.1 146.7) (end 117.2 146.8) (width 0.8) (layer "F.Cu") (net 7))
 (segment (start 119.575 139.455) (end 118.145 139.455) (width 0.8) (layer "F.Cu") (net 7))
 (segment (start 117.2 148) (end 117.2 146.8) (width 0.8) (layer "F.Cu") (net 7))
 (segment (start 117.2 145.4) (end 117.2 144.6) (width 0.8) (layer "F.Cu") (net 7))
 (segment (start 108.935 145.335) (end 110.3 146.7) (width 0.8) (layer "F.Cu") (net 7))
 (segment (start 100.775 135.175) (end 100.775 137.715) (width 0.8) (layer "F.Cu") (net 1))
 (segment (start 100.775 137.715) (end 108.395 137.715) (width 0.8) (layer "F.Cu") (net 1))
 (segment (start 108.395 137.715) (end 112.485 137.715) (width 0.8) (layer "F.Cu") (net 1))
 (segment (start 112.485 137.715) (end 115.2 135) (width 0.8) (layer "F.Cu") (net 1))
 (segment (start 107.275 147.875) (end 108.395 147.875) (width 0.8) (layer "F.Cu") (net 3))
 (segment (start 100.775 142.795) (end 102.195 142.795) (width 0.8) (layer "F.Cu") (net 3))
 (segment (start 108.395 150.415) (end 108.395 147.875) (width 0.8) (layer "F.Cu") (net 3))
 (segment (start 102.195 142.795) (end 107.275 147.875) (width 0.8) (layer "F.Cu") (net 3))
 (segment (start 112.6 143.1) (end 112.6 141.22) (width 0.8) (layer "F.Cu") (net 9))
 (segment (start 113.275 140.255) (end 113.42 140.4) (width 0.8) (layer "F.Cu") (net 9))
 (segment (start 108.395 140.255) (end 113.275 140.255) (width 0.8) (layer "F.Cu") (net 9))
 (segment (start 112.6 141.22) (end 113.42 140.4) (width 0.8) (layer "F.Cu") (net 9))
 (segment (start 125.745 139.455) (end 127.195 139.455) (width 0.8) (layer "F.Cu") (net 12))
 (segment (start 125.335 144.535) (end 125.2 144.4) (width 0.8) (layer "F.Cu") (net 12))
 (segment (start 125.2 153.2) (end 125.2 144.4) (width 0.8) (layer "F.Cu") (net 12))
 (segment (start 125.2 144.4) (end 125.2 140) (width 0.8) (layer "F.Cu") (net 12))
 (segment (start 125.2 140) (end 125.745 139.455) (width 0.8) (layer "F.Cu") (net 12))
 (segment (start 127.195 144.535) (end 125.335 144.535) (width 0.8) (layer "F.Cu") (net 12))
 (segment (start 121.8 147.2) (end 121.8 142) (width 0.8) (layer "F.Cu") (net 11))
 (segment (start 119.575 136.915) (end 121.115 136.915) (width 0.8) (layer "F.Cu") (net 11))
 (segment (start 119.575 147.075) (end 121.675 147.075) (width 0.8) (layer "F.Cu") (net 11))
 (segment (start 121.8 152.8) (end 121.8 147.2) (width 0.8) (layer "F.Cu") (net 11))
 (segment (start 121.795 141.995) (end 121.8 142) (width 0.8) (layer "F.Cu") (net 11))
 (segment (start 119.575 141.995) (end 121.795 141.995) (width 0.8) (layer "F.Cu") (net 11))
 (segment (start 121.115 136.915) (end 121.8 137.6) (width 0.8) (layer "F.Cu") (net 11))
 (segment (start 121.4 153.2) (end 121.8 152.8) (width 0.8) (layer "F.Cu") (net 11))
 (segment (start 121.8 142) (end 121.8 137.6) (width 0.8) (layer "F.Cu") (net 11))
 (segment (start 121.675 147.075) (end 121.8 147.2) (width 0.8) (layer "F.Cu") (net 11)))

